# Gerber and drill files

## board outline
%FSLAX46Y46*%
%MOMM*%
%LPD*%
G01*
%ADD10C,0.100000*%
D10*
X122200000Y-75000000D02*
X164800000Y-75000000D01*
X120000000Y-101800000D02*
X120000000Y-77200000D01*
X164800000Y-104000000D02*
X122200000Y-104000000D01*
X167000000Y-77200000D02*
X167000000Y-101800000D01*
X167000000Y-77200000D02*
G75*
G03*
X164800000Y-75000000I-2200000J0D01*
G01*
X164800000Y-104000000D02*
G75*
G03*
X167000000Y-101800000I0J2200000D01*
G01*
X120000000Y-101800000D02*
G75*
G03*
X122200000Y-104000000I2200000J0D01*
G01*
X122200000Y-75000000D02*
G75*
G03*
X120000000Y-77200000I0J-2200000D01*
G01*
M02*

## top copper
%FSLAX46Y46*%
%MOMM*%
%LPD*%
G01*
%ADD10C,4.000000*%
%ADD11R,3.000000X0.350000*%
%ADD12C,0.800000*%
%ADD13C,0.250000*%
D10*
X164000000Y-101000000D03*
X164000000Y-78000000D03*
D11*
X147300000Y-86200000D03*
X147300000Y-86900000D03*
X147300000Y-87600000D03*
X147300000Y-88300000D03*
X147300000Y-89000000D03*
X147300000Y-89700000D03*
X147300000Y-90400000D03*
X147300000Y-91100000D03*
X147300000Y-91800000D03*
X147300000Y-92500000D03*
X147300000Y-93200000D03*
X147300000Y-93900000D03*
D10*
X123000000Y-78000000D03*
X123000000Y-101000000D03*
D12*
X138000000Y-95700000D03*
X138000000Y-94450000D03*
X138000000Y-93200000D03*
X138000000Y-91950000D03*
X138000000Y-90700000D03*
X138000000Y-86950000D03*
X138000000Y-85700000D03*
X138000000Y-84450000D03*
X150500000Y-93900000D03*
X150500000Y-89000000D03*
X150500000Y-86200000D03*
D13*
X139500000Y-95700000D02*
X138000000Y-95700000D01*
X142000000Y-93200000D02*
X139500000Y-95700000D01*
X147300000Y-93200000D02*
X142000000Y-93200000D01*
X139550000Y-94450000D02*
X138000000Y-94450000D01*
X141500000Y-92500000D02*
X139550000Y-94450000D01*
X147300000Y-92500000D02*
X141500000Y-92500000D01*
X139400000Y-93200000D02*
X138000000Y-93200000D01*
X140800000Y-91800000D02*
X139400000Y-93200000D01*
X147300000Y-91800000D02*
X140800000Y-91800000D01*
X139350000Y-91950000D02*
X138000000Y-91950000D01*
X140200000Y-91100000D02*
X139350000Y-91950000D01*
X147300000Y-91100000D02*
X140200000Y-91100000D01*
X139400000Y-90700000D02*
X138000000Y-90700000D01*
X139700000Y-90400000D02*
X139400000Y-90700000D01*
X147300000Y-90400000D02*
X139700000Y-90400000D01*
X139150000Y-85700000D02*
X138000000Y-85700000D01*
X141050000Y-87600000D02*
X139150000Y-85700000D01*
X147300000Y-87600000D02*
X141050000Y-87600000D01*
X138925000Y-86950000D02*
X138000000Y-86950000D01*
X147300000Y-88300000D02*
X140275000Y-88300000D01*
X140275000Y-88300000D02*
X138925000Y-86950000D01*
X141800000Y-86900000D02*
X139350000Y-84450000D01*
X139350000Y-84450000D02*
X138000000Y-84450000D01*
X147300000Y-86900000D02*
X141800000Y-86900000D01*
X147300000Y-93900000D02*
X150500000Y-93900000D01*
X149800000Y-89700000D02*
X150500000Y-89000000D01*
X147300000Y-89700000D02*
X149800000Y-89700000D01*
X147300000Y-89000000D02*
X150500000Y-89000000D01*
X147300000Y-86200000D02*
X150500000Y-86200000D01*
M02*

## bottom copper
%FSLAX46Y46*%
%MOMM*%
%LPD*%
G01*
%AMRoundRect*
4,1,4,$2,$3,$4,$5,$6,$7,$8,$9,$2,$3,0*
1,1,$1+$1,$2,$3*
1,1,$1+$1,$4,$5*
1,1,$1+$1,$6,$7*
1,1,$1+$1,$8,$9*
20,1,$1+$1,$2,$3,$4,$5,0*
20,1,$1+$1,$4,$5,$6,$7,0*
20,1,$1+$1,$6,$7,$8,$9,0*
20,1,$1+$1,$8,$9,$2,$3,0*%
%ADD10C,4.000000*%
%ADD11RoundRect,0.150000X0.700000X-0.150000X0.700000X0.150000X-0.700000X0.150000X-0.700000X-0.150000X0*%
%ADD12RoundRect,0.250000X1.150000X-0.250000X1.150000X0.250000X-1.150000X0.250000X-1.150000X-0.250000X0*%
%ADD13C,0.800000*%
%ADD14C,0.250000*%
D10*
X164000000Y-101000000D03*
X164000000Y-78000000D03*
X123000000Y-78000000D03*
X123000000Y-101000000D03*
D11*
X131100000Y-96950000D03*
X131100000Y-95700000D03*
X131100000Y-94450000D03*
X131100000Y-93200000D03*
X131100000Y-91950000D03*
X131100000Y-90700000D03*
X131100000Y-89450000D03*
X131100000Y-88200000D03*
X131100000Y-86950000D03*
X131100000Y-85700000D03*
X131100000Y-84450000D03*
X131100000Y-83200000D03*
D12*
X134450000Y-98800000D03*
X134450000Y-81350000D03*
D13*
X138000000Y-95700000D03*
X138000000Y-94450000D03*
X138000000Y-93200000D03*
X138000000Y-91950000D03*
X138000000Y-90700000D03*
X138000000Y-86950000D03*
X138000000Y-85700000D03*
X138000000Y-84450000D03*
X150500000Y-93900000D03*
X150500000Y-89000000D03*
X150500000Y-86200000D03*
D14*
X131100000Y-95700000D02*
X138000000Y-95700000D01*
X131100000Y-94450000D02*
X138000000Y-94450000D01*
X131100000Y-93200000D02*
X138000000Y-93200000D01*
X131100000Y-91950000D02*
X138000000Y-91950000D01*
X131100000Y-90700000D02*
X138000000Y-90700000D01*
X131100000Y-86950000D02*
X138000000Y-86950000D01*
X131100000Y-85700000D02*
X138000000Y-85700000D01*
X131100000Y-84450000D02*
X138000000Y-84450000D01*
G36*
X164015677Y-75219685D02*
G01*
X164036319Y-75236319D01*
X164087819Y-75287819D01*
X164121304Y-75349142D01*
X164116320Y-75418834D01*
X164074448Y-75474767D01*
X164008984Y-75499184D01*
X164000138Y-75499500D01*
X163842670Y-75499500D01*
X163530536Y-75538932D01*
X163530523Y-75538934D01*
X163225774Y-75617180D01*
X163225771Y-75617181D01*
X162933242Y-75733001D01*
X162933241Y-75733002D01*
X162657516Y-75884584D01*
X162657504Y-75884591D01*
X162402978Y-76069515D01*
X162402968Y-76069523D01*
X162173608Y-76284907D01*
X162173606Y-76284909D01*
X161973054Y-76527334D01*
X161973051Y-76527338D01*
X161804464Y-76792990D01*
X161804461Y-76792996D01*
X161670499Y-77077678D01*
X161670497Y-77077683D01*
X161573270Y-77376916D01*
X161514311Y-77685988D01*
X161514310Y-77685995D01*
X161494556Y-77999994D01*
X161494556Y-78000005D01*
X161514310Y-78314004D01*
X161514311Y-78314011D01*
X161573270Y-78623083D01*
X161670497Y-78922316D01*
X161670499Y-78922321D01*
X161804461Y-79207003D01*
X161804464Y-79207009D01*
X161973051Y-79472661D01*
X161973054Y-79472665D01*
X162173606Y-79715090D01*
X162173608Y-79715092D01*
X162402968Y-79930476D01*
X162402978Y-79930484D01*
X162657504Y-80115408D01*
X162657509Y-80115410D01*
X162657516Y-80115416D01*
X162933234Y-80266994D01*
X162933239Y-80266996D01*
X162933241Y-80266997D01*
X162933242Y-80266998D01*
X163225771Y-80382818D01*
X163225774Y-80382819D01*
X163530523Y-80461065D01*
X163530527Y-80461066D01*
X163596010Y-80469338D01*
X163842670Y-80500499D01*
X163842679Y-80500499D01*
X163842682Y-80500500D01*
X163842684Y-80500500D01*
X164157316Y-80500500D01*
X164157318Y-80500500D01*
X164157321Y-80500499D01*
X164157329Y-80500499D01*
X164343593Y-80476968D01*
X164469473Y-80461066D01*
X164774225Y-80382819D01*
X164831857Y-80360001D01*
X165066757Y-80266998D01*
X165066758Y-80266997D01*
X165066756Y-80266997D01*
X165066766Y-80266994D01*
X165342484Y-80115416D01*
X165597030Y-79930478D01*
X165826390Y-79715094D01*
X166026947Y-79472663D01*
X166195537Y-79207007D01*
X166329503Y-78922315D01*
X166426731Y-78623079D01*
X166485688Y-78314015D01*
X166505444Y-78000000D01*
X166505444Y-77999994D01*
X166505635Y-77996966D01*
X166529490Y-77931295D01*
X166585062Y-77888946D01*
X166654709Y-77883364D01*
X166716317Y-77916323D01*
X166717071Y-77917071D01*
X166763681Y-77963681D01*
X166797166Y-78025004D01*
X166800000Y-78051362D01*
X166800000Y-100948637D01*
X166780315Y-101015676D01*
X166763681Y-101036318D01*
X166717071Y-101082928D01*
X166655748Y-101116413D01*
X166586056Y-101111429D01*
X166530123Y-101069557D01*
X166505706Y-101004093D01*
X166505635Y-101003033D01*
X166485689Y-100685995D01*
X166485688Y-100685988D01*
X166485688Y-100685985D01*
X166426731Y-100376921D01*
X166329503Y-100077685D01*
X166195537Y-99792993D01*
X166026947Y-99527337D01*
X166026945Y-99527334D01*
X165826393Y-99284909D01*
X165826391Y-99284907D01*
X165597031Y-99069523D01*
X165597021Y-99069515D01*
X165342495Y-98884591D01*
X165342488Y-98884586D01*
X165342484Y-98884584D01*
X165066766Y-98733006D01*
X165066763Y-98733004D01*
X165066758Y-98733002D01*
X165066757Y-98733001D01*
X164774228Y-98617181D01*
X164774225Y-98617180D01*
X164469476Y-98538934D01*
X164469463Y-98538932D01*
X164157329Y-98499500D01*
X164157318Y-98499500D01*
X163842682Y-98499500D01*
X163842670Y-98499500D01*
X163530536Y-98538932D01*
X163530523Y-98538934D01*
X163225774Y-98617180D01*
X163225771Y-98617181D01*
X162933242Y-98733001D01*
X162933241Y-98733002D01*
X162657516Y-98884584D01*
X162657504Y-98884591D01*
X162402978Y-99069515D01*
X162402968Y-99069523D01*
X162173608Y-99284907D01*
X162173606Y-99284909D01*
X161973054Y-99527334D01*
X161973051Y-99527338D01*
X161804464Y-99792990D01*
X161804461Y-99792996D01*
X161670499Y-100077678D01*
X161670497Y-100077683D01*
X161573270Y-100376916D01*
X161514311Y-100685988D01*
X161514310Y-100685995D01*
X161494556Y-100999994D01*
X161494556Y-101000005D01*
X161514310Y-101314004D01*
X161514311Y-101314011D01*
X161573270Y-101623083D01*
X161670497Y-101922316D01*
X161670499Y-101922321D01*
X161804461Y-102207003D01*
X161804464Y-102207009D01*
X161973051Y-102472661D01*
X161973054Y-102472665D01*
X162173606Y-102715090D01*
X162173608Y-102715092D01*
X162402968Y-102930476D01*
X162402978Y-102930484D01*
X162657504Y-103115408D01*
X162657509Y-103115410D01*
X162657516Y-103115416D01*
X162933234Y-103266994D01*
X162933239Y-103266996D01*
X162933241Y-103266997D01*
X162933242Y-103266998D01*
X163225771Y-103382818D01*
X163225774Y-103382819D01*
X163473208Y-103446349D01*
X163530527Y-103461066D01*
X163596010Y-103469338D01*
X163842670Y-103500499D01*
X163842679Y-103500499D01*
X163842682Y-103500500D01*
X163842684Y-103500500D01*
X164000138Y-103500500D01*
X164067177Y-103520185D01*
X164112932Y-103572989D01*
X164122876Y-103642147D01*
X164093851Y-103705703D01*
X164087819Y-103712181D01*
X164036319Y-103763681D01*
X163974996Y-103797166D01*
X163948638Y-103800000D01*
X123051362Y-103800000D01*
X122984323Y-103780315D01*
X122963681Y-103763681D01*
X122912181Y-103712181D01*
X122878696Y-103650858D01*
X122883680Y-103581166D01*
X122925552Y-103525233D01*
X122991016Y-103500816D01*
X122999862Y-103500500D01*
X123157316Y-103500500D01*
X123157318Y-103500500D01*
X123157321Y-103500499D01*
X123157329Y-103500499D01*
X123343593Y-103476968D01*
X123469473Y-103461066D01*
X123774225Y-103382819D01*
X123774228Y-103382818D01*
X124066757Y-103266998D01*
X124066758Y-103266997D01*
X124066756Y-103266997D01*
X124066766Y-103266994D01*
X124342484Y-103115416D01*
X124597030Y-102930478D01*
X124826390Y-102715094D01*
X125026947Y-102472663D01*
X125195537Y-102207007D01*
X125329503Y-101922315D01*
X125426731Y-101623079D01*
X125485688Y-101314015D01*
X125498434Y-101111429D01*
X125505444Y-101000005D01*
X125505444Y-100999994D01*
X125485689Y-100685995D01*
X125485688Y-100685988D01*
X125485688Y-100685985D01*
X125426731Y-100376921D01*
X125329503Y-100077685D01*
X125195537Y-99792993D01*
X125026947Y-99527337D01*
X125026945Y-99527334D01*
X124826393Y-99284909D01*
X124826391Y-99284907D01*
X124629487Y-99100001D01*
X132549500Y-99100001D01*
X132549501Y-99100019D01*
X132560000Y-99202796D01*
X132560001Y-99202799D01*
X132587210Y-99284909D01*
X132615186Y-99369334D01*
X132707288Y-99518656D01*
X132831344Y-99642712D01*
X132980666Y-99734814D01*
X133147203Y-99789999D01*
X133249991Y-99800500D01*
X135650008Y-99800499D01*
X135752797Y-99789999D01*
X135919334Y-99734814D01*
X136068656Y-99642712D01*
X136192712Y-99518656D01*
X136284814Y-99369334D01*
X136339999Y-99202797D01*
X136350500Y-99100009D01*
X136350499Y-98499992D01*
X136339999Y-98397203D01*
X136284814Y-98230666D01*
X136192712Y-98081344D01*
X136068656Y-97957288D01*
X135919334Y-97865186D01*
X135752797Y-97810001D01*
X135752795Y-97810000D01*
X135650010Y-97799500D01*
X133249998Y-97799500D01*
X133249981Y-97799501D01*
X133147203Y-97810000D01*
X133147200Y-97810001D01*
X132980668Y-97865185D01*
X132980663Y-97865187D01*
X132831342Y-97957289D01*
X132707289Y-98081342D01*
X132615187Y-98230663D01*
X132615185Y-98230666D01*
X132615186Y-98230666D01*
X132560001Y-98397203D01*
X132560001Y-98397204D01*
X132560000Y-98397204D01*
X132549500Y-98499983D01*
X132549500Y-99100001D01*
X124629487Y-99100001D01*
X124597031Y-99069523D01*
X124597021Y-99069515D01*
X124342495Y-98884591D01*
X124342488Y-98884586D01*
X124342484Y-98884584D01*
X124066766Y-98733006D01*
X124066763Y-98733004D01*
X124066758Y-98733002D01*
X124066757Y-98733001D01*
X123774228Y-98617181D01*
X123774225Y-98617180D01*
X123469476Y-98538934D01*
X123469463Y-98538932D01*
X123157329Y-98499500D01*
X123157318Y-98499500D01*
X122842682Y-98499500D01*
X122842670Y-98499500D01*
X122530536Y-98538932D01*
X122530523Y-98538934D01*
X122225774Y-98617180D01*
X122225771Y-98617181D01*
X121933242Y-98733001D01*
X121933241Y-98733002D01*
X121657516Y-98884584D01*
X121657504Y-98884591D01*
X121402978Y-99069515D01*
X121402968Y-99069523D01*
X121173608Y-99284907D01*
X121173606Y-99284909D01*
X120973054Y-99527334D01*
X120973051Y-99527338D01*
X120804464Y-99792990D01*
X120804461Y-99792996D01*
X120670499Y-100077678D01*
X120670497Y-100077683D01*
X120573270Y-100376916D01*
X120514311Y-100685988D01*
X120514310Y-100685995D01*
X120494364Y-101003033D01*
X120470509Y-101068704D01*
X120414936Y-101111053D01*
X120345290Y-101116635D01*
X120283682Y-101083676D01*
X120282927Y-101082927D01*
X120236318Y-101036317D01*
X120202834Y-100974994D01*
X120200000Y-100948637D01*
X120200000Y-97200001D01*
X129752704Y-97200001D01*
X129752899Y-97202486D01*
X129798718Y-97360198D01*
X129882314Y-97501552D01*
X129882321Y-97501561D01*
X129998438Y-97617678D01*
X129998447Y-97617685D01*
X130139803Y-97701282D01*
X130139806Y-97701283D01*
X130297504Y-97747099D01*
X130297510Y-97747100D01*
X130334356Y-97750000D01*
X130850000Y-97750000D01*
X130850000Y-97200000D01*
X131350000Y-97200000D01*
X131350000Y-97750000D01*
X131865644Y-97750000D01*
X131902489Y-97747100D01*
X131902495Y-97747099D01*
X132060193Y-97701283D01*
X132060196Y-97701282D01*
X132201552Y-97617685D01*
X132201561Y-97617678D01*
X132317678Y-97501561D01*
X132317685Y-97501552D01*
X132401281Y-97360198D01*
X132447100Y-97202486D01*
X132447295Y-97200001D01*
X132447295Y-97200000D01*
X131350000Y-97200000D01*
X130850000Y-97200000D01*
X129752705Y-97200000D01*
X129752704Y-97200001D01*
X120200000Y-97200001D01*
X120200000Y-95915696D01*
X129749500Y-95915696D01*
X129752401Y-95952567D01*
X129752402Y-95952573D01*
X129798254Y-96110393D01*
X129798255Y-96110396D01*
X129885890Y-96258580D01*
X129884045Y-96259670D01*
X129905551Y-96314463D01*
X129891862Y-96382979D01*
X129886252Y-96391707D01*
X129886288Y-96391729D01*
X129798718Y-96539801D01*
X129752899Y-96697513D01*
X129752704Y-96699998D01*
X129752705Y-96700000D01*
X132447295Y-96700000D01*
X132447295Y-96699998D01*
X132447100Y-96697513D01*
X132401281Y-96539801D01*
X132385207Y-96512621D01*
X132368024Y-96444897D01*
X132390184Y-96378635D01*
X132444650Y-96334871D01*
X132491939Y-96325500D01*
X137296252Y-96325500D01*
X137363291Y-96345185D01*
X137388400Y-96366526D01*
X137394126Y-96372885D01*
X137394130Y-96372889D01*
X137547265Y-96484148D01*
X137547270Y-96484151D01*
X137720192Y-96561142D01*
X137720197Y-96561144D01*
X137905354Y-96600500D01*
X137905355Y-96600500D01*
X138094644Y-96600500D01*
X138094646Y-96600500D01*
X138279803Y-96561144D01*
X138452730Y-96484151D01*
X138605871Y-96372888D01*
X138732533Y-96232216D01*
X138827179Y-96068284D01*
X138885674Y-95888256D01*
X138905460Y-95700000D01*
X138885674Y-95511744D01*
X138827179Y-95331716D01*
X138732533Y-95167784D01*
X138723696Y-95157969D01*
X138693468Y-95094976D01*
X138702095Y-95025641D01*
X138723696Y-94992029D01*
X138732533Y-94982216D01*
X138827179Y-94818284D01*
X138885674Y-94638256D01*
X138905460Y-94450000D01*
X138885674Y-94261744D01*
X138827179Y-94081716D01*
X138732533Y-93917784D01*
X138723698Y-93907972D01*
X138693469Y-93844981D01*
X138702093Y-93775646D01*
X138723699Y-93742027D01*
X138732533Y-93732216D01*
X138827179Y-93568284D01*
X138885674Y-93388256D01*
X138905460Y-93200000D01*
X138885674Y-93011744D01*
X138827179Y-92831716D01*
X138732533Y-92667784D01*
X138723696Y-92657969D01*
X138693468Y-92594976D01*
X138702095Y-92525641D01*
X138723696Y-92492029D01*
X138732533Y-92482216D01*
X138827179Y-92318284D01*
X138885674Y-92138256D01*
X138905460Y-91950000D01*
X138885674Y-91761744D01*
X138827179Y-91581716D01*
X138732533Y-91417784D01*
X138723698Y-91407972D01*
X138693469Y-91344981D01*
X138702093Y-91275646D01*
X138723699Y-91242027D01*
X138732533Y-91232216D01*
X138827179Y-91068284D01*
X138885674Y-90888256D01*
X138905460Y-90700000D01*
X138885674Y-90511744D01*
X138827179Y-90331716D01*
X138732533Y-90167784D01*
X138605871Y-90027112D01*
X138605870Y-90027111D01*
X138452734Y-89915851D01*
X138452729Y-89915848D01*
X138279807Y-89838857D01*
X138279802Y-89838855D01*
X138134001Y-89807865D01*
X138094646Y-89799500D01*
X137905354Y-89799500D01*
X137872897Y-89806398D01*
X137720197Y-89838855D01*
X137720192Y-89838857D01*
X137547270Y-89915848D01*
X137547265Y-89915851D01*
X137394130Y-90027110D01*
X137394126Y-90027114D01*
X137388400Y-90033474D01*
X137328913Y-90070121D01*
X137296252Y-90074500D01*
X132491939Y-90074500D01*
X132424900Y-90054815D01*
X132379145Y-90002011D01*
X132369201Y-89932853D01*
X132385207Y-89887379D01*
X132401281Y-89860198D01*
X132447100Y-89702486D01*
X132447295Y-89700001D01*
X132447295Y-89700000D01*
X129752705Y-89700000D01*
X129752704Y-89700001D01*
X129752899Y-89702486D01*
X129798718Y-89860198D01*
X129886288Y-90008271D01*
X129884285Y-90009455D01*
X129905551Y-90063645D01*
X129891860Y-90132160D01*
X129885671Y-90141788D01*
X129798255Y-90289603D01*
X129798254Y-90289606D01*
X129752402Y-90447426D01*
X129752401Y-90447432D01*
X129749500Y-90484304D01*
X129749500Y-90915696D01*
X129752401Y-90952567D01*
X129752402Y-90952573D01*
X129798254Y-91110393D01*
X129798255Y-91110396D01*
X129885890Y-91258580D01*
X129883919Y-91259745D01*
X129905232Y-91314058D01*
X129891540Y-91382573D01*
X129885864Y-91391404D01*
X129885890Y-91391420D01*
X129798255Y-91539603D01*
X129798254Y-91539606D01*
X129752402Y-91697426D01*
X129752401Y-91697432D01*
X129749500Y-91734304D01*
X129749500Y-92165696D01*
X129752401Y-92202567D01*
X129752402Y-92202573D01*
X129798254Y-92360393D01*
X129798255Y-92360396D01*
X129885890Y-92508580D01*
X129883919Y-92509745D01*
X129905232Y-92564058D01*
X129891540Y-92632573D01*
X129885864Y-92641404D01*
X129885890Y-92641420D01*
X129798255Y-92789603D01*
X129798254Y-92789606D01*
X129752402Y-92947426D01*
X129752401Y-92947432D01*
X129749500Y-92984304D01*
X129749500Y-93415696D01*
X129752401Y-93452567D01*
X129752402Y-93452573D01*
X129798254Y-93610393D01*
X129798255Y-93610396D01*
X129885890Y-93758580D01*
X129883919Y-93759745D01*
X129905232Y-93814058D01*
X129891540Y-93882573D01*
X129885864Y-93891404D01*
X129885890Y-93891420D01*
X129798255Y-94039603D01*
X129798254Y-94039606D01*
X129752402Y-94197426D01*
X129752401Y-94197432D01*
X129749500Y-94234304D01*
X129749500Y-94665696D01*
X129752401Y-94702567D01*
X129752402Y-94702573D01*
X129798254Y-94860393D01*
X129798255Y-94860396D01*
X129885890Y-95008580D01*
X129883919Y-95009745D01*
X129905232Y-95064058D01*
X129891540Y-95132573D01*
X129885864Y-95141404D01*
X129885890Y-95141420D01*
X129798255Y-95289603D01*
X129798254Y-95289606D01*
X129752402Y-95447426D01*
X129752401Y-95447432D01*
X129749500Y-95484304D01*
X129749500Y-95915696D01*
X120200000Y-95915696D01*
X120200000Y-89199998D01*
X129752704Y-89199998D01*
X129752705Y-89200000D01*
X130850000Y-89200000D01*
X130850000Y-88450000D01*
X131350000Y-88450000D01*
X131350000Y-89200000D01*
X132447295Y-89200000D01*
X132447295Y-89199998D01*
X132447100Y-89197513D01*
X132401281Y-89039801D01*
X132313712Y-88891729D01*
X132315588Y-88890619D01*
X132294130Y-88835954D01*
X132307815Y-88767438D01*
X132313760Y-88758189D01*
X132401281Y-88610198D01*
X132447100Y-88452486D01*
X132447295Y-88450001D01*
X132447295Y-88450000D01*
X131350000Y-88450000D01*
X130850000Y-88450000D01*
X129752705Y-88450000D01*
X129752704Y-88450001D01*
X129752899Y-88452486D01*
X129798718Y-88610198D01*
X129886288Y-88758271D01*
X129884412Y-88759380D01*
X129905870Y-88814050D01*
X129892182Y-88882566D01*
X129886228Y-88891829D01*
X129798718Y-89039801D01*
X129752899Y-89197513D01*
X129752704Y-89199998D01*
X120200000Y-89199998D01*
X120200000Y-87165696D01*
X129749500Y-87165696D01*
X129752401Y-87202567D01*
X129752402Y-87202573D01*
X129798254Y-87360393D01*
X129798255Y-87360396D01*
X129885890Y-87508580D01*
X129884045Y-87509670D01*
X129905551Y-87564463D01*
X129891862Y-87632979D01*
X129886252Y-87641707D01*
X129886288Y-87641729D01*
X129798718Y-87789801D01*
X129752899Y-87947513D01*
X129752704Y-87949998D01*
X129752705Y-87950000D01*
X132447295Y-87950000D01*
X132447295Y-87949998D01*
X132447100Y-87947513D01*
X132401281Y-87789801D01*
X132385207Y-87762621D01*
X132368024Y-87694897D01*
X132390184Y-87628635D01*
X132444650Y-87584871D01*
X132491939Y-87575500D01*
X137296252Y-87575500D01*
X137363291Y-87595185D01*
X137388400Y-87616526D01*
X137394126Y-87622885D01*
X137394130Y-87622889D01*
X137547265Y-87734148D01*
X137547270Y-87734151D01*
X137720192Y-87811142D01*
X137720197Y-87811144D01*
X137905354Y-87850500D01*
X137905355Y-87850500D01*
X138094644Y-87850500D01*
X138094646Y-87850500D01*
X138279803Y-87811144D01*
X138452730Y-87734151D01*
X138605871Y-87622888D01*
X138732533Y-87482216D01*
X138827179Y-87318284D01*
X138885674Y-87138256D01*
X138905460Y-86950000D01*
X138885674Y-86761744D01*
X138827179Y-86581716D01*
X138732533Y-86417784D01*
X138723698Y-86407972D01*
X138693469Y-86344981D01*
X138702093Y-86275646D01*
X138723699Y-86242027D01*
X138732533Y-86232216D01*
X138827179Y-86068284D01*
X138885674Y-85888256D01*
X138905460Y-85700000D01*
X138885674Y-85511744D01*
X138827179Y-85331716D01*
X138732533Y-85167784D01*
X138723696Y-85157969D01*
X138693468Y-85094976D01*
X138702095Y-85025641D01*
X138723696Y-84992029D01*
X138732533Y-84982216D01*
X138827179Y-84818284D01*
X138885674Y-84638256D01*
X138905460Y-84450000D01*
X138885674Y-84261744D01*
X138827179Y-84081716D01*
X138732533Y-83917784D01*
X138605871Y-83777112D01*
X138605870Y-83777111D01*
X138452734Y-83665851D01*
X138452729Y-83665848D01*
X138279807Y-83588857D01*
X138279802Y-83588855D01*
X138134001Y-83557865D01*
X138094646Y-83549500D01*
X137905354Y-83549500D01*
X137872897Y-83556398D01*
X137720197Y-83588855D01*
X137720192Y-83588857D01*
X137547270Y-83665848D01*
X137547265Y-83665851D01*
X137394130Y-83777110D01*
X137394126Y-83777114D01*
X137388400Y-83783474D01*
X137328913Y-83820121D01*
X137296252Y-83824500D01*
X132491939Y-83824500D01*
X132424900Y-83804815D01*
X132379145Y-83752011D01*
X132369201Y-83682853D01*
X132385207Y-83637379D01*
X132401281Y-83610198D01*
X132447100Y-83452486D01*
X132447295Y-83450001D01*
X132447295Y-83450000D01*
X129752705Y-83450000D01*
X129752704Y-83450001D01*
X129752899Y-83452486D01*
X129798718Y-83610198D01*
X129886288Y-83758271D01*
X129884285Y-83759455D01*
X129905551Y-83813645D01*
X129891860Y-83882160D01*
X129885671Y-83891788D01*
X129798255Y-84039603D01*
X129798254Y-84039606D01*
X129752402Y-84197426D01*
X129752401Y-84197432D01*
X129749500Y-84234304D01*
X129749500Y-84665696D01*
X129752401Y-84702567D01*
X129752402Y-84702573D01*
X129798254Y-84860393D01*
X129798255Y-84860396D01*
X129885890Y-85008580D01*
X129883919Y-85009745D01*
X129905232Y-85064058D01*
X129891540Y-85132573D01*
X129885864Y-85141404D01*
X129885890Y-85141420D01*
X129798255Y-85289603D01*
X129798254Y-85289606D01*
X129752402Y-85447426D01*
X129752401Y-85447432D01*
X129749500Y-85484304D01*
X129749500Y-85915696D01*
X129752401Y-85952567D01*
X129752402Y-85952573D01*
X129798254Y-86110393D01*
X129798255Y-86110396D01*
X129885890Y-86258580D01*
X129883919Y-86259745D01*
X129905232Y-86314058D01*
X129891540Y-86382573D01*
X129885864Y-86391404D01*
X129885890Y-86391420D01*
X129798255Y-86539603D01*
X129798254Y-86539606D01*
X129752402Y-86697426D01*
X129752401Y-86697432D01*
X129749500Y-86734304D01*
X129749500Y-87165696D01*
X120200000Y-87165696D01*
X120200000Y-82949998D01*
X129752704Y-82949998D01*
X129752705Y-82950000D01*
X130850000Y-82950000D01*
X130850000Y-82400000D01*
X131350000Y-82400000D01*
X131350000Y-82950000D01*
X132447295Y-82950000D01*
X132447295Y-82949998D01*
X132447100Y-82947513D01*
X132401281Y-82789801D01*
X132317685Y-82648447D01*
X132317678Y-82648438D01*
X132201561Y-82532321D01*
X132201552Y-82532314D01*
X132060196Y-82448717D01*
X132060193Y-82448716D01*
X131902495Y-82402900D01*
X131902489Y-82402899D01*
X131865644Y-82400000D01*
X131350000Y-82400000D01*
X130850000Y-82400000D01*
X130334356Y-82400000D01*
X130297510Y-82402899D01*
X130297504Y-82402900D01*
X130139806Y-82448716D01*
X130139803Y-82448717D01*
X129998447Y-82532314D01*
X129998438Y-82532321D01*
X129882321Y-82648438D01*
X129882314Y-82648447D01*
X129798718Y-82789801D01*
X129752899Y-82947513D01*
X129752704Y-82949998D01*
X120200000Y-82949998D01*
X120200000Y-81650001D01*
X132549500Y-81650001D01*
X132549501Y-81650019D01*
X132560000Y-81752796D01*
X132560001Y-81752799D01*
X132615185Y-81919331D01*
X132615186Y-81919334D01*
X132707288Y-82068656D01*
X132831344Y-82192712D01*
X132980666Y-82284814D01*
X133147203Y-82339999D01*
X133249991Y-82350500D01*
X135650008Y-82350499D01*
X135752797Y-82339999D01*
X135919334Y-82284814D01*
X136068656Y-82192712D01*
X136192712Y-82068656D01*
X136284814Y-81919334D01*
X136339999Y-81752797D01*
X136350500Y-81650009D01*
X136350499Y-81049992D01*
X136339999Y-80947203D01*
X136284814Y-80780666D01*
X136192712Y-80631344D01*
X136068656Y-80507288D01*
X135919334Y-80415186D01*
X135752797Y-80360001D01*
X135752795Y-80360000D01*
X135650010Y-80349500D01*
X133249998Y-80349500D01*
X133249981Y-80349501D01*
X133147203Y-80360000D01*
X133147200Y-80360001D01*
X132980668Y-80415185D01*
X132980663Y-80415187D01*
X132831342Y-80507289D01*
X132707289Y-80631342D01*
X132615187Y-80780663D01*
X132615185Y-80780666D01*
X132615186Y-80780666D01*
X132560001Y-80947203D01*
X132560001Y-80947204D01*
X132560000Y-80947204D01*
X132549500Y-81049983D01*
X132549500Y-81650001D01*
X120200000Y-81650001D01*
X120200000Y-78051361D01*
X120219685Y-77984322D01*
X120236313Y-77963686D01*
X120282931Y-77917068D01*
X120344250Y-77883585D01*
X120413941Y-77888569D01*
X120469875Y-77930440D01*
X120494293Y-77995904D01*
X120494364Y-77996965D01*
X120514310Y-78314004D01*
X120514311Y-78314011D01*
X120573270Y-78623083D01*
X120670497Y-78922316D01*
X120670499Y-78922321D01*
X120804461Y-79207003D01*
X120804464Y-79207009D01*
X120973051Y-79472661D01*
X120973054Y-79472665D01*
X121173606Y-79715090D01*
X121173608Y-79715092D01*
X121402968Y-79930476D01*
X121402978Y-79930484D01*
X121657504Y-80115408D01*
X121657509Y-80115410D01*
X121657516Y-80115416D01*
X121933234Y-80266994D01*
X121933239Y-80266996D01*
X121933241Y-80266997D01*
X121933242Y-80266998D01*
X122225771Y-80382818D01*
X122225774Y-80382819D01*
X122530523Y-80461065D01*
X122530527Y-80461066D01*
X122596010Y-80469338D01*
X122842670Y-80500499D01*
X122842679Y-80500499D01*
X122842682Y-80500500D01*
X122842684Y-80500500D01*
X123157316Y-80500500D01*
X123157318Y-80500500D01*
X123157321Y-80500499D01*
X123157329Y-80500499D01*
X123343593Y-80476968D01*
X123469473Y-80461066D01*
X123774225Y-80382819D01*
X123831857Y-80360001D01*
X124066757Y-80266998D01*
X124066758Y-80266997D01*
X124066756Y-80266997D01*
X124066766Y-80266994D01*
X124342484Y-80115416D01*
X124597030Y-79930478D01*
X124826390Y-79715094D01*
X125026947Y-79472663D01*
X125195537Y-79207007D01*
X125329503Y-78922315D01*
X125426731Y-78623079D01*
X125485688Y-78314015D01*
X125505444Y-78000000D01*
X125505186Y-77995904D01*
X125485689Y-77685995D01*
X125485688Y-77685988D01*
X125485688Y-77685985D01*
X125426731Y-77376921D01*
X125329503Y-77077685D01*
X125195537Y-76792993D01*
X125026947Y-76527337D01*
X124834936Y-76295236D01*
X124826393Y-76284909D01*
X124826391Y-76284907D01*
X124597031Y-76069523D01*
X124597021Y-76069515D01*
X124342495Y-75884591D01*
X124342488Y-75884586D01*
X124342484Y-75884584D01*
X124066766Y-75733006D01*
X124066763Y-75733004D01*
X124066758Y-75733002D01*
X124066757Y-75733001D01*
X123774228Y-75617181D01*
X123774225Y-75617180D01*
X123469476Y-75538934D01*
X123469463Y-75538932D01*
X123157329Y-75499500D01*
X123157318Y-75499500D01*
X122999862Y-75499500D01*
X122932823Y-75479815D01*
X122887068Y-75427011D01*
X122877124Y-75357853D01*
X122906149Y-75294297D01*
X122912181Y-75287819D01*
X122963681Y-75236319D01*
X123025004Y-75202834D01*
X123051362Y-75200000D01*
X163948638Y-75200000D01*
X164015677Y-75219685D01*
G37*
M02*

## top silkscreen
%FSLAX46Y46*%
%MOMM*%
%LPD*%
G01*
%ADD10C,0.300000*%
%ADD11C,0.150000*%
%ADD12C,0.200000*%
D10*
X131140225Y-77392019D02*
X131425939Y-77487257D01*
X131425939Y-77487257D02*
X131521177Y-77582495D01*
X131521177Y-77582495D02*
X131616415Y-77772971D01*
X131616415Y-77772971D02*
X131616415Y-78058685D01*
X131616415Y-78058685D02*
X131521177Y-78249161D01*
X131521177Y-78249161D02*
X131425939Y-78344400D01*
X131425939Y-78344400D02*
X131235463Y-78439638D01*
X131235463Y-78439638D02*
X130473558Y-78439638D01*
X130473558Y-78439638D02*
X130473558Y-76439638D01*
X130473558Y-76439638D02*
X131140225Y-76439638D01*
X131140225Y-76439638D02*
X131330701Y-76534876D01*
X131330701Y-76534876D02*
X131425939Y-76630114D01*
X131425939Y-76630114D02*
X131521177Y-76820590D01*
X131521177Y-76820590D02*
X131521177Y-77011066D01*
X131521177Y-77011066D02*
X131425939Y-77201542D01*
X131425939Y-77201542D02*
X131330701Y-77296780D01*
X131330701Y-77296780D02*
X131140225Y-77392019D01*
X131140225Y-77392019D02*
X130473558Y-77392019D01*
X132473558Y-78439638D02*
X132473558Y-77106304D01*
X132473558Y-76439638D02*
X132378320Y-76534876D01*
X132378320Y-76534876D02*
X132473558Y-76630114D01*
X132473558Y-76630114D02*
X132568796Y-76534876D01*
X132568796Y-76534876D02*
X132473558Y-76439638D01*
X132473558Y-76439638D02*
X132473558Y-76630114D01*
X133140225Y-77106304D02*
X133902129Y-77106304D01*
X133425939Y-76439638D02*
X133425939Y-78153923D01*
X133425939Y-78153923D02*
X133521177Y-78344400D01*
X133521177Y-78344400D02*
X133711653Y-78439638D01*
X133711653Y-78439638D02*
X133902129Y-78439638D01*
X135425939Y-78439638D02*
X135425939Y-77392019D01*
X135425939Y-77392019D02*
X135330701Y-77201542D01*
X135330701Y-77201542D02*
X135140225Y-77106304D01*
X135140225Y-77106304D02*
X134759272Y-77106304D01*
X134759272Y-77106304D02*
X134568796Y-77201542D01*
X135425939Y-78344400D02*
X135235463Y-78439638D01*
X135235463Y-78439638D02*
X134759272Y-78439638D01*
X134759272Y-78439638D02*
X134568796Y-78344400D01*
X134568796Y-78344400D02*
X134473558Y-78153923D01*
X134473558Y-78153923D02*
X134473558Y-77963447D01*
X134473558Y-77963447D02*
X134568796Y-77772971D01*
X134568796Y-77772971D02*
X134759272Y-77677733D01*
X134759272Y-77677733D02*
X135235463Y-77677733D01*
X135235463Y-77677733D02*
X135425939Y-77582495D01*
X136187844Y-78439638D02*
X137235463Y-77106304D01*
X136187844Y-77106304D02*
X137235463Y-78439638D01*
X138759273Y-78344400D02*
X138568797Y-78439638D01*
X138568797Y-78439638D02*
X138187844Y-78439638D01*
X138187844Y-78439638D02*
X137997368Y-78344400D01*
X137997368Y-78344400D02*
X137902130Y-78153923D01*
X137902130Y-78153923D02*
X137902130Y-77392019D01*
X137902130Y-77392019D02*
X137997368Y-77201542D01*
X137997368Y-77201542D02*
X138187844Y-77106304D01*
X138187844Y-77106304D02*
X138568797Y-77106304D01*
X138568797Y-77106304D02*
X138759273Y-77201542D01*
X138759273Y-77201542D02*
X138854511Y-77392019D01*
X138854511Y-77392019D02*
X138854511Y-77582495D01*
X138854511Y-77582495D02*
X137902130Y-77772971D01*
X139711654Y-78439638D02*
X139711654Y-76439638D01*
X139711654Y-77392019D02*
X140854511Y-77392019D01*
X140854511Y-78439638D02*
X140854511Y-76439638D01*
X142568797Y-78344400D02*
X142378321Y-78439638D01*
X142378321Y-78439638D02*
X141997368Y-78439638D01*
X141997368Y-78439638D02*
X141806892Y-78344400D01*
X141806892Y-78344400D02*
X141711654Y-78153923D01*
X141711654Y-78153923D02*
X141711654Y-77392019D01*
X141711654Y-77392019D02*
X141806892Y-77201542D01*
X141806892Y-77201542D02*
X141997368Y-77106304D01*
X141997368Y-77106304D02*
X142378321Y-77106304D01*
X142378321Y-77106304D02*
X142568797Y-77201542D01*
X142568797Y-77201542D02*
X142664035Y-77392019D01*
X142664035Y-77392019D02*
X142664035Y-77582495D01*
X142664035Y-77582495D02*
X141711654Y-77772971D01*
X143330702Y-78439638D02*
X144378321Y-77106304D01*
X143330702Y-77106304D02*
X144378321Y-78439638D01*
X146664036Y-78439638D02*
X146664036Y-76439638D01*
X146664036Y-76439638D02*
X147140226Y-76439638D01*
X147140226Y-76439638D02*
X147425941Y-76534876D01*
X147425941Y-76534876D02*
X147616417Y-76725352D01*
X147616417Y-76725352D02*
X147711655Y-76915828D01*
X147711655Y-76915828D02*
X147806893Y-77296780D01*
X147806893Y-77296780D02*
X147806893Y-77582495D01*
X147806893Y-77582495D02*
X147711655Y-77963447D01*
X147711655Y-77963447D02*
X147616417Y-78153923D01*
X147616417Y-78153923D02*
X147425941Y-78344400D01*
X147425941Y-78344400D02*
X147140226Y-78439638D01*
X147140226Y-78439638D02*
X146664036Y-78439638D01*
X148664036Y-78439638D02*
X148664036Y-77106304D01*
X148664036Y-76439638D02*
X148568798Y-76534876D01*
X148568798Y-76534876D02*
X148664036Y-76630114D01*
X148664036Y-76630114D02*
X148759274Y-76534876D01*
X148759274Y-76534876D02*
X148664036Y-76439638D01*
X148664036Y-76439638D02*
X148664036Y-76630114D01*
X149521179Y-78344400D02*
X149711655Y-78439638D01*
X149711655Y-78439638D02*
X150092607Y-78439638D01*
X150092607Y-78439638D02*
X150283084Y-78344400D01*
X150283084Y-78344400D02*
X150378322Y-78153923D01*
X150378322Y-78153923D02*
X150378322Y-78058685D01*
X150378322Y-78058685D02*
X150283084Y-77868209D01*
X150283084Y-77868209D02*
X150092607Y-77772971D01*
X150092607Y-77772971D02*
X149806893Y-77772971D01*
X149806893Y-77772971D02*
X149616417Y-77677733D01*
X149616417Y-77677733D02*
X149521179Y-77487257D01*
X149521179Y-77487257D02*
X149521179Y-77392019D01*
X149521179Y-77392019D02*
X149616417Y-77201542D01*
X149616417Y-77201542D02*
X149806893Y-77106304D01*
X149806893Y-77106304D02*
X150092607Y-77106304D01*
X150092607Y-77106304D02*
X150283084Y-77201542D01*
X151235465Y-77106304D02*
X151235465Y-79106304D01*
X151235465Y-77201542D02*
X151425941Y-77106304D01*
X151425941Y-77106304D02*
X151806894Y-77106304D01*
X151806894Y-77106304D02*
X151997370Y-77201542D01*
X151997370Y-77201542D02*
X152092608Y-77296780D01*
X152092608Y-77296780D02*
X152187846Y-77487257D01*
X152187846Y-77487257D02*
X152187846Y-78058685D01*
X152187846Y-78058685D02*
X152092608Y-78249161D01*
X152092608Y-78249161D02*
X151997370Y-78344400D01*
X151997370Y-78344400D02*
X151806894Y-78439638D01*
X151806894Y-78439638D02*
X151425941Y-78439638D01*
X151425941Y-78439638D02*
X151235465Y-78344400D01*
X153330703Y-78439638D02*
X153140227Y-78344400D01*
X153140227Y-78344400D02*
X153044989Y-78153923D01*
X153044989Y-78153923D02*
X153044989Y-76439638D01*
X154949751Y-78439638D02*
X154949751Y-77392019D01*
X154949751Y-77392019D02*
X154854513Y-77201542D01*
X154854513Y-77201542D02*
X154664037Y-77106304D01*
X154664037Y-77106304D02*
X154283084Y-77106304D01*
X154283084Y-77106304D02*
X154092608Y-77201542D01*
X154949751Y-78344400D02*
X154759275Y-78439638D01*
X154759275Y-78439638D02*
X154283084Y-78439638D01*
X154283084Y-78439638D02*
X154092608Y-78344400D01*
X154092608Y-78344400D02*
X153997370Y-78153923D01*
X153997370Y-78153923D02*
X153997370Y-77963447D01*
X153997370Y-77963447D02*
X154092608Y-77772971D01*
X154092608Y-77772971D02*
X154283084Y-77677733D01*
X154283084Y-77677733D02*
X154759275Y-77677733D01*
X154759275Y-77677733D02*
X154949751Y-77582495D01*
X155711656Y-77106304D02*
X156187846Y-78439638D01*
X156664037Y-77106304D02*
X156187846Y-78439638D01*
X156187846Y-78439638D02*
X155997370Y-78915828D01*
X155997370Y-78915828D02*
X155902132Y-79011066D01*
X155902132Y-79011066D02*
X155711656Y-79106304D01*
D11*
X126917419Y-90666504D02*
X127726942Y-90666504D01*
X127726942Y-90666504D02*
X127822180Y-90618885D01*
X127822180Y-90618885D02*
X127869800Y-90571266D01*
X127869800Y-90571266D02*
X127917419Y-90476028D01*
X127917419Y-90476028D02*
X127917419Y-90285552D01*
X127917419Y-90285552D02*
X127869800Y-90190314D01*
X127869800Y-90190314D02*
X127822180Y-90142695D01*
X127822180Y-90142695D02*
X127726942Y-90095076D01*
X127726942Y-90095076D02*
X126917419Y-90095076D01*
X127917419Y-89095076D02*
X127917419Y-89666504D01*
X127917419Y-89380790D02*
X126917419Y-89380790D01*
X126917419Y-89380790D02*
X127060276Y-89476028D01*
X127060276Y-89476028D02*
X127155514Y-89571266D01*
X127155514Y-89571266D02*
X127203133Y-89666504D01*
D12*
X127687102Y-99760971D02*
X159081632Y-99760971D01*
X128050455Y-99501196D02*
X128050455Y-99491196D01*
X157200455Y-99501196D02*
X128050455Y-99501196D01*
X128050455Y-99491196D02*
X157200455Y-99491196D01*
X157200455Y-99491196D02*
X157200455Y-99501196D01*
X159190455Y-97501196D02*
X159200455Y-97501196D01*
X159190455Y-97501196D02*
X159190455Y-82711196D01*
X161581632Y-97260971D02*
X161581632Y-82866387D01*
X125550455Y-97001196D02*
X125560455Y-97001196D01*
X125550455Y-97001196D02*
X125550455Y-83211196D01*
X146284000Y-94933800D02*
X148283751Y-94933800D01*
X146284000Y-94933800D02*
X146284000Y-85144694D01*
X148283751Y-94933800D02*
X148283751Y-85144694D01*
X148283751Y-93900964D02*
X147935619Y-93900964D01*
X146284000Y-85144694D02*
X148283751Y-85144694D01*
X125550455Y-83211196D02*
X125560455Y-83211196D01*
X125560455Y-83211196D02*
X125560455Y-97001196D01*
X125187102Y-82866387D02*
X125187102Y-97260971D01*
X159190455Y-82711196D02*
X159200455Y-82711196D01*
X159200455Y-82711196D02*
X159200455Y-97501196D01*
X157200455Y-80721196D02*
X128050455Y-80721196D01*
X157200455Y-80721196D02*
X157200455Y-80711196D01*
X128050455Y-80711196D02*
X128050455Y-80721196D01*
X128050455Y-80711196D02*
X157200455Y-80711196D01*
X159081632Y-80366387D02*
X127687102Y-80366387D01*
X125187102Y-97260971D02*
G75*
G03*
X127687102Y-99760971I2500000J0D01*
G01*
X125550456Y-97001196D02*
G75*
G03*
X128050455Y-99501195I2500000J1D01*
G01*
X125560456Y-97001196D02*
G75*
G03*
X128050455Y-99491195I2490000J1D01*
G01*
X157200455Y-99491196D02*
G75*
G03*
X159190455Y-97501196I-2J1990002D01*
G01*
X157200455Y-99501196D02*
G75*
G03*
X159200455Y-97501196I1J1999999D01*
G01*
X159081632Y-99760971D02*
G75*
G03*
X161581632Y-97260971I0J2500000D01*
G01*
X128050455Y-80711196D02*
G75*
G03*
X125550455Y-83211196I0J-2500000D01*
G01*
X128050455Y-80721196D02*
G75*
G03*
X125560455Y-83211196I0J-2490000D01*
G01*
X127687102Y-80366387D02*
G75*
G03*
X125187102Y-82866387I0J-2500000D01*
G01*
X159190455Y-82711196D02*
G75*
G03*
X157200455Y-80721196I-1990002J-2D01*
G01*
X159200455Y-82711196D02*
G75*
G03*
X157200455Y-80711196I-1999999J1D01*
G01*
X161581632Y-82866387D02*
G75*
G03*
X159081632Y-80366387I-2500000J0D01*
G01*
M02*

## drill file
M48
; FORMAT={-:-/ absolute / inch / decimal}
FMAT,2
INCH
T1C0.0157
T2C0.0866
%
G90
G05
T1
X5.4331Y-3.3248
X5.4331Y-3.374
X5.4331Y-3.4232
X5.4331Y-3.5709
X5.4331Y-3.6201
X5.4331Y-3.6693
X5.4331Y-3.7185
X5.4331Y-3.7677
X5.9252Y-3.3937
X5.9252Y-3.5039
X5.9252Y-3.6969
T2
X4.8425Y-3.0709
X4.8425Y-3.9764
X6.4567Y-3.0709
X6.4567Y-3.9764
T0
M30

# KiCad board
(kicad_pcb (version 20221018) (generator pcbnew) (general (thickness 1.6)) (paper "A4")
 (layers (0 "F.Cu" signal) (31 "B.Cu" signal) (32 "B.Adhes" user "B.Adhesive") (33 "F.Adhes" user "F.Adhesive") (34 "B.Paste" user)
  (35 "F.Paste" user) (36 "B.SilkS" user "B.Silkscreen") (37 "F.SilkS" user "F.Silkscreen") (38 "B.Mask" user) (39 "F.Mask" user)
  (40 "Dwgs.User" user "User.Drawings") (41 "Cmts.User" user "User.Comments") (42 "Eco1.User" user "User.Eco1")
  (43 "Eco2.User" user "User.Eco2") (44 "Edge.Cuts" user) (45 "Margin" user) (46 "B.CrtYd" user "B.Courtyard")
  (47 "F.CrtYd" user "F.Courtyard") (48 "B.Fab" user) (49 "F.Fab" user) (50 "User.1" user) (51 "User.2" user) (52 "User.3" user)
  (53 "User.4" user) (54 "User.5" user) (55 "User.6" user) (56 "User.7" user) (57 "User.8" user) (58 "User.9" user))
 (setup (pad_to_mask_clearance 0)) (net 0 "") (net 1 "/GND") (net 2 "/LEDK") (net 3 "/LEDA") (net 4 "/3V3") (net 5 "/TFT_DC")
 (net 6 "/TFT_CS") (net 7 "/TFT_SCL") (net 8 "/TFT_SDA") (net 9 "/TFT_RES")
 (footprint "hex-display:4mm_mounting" (layer "F.Cu") (at 164.1 101.2)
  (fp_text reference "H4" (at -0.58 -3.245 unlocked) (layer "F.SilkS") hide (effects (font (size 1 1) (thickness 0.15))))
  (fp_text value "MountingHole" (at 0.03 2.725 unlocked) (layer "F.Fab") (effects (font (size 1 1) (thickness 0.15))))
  (pad "" thru_hole circle (at -0.1 -0.2) (size 4 4) (drill 2.2) (layers "*.Cu" "*.Mask") (zone_connect 0)))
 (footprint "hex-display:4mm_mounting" (layer "F.Cu") (at 163.6 78.2)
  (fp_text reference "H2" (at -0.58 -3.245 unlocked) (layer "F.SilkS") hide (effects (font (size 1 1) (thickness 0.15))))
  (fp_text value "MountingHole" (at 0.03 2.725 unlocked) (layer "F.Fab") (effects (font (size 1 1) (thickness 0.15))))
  (pad "" thru_hole circle (at 0.4 -0.2) (size 4 4) (drill 2.2) (layers "*.Cu" "*.Mask") (zone_connect 0)))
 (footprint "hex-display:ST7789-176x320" (layer "F.Cu") (at 172.954 65.7238 90)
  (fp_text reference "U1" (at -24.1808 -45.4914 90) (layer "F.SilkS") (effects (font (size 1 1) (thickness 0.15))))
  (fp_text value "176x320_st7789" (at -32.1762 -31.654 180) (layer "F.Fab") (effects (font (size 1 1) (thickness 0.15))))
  (fp_line (start -34.037171 -45.266898) (end -34.037171 -13.872368) (stroke (width 0.2) (type solid)) (layer "F.SilkS"))
  (fp_line (start -33.777396 -44.903545) (end -33.767396 -44.903545) (stroke (width 0.2) (type solid)) (layer "F.SilkS"))
  (fp_line (start -33.777396 -15.753545) (end -33.777396 -44.903545) (stroke (width 0.2) (type solid)) (layer "F.SilkS"))
  (fp_line (start -33.767396 -44.903545) (end -33.767396 -15.753545) (stroke (width 0.2) (type solid)) (layer "F.SilkS"))
  (fp_line (start -33.767396 -15.753545) (end -33.777396 -15.753545) (stroke (width 0.2) (type solid)) (layer "F.SilkS"))
  (fp_line (start -31.777396 -13.763545) (end -31.777396 -13.753545) (stroke (width 0.2) (type solid)) (layer "F.SilkS"))
  (fp_line (start -31.777396 -13.763545) (end -16.987396 -13.763545) (stroke (width 0.2) (type solid)) (layer "F.SilkS"))
  (fp_line (start -31.537171 -11.372368) (end -17.142587 -11.372368) (stroke (width 0.2) (type solid)) (layer "F.SilkS"))
  (fp_line (start -31.277396 -47.403545) (end -31.277396 -47.393545) (stroke (width 0.2) (type solid)) (layer "F.SilkS"))
  (fp_line (start -31.277396 -47.403545) (end -17.487396 -47.403545) (stroke (width 0.2) (type solid)) (layer "F.SilkS"))
  (fp_line (start -29.21 -26.67) (end -29.21 -24.670249) (stroke (width 0.2) (type solid)) (layer "F.SilkS"))
  (fp_line (start -29.21 -26.67) (end -19.420894 -26.67) (stroke (width 0.2) (type solid)) (layer "F.SilkS"))
  (fp_line (start -29.21 -24.670249) (end -19.420894 -24.670249) (stroke (width 0.2) (type solid)) (layer "F.SilkS"))
  (fp_line (start -28.177164 -24.670249) (end -28.177164 -25.018381) (stroke (width 0.2) (type solid)) (layer "F.SilkS"))
  (fp_line (start -19.420894 -26.67) (end -19.420894 -24.670249) (stroke (width 0.2) (type solid)) (layer "F.SilkS"))
  (fp_line (start -17.487396 -47.403545) (end -17.487396 -47.393545) (stroke (width 0.2) (type solid)) (layer "F.SilkS"))
  (fp_line (start -17.487396 -47.393545) (end -31.277396 -47.393545) (stroke (width 0.2) (type solid)) (layer "F.SilkS"))
  (fp_line (start -17.142587 -47.766898) (end -31.537171 -47.766898) (stroke (width 0.2) (type solid)) (layer "F.SilkS"))
  (fp_line (start -16.987396 -13.763545) (end -16.987396 -13.753545) (stroke (width 0.2) (type solid)) (layer "F.SilkS"))
  (fp_line (start -16.987396 -13.753545) (end -31.777396 -13.753545) (stroke (width 0.2) (type solid)) (layer "F.SilkS"))
  (fp_line (start -14.997396 -15.753545) (end -14.997396 -44.903545) (stroke (width 0.2) (type solid)) (layer "F.SilkS"))
  (fp_line (start -14.997396 -15.753545) (end -14.987396 -15.753545) (stroke (width 0.2) (type solid)) (layer "F.SilkS"))
  (fp_line (start -14.987396 -44.903545) (end -14.997396 -44.903545) (stroke (width 0.2) (type solid)) (layer "F.SilkS"))
  (fp_line (start -14.987396 -44.903545) (end -14.987396 -15.753545) (stroke (width 0.2) (type solid)) (layer "F.SilkS"))
  (fp_line (start -14.642587 -13.872368) (end -14.642587 -45.266898) (stroke (width 0.2) (type solid)) (layer "F.SilkS"))
  (fp_arc (start -34.037171 -45.266898) (mid -33.304938 -47.034665) (end -31.537171 -47.766898) (stroke (width 0.2) (type solid))
   (layer "F.SilkS"))
  (fp_arc (start -33.777395 -44.903545) (mid -33.045162 -46.671311) (end -31.277396 -47.403544) (stroke (width 0.2) (type solid))
   (layer "F.SilkS"))
  (fp_arc (start -33.767395 -44.903545) (mid -33.038091 -46.66424) (end -31.277396 -47.393544) (stroke (width 0.2) (type solid))
   (layer "F.SilkS"))
  (fp_arc (start -31.777396 -13.763545) (mid -33.184538 -14.346403) (end -33.767396 -15.753545) (stroke (width 0.2) (type solid))
   (layer "F.SilkS"))
  (fp_arc (start -31.777396 -13.753545) (mid -33.19161 -14.339331) (end -33.777396 -15.753545) (stroke (width 0.2) (type solid))
   (layer "F.SilkS"))
  (fp_arc (start -31.537171 -11.372368) (mid -33.304938 -12.104601) (end -34.037171 -13.872368) (stroke (width 0.2) (type solid))
   (layer "F.SilkS"))
  (fp_arc (start -17.487396 -47.403545) (mid -15.719629 -46.671312) (end -14.987396 -44.903545) (stroke (width 0.2) (type solid))
   (layer "F.SilkS"))
  (fp_arc (start -17.487396 -47.393545) (mid -15.7267 -46.664241) (end -14.997396 -44.903545) (stroke (width 0.2) (type solid))
   (layer "F.SilkS"))
  (fp_arc (start -17.142587 -47.766898) (mid -15.37482 -47.034665) (end -14.642587 -45.266898) (stroke (width 0.2) (type solid))
   (layer "F.SilkS"))
  (fp_arc (start -14.997396 -15.753545) (mid -15.580254 -14.346403) (end -16.987396 -13.763545) (stroke (width 0.2) (type solid))
   (layer "F.SilkS"))
  (fp_arc (start -14.987396 -15.753545) (mid -15.573182 -14.339331) (end -16.987396 -13.753545) (stroke (width 0.2) (type solid))
   (layer "F.SilkS"))
  (fp_arc (start -14.642587 -13.872368) (mid -15.37482 -12.104601) (end -17.142587 -11.372368) (stroke (width 0.2) (type solid))
   (layer "F.SilkS"))
  (pad "1" smd rect (at -20.4762 -25.654 270) (size 0.35 3) (layers "F.Cu" "F.Paste" "F.Mask") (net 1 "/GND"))
  (pad "2" smd rect (at -21.1762 -25.654 270) (size 0.35 3) (layers "F.Cu" "F.Paste" "F.Mask") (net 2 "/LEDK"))
  (pad "3" smd rect (at -21.8762 -25.654 270) (size 0.35 3) (layers "F.Cu" "F.Paste" "F.Mask") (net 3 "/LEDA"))
  (pad "4" smd rect (at -22.5762 -25.654 270) (size 0.35 3) (layers "F.Cu" "F.Paste" "F.Mask") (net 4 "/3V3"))
  (pad "5" smd rect (at -23.2762 -25.654 270) (size 0.35 3) (layers "F.Cu" "F.Paste" "F.Mask") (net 1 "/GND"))
  (pad "6" smd rect (at -23.9762 -25.654 270) (size 0.35 3) (layers "F.Cu" "F.Paste" "F.Mask") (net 1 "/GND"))
  (pad "7" smd rect (at -24.6762 -25.654 270) (size 0.35 3) (layers "F.Cu" "F.Paste" "F.Mask") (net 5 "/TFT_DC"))
  (pad "8" smd rect (at -25.3762 -25.654 270) (size 0.35 3) (layers "F.Cu" "F.Paste" "F.Mask") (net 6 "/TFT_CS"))
  (pad "9" smd rect (at -26.0762 -25.654 270) (size 0.35 3) (layers "F.Cu" "F.Paste" "F.Mask") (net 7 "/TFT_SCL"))
  (pad "10" smd rect (at -26.7762 -25.654 270) (size 0.35 3) (layers "F.Cu" "F.Paste" "F.Mask") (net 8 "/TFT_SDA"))
  (pad "11" smd rect (at -27.4762 -25.654 270) (size 0.35 3) (layers "F.Cu" "F.Paste" "F.Mask") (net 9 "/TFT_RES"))
  (pad "12" smd rect (at -28.1762 -25.654 270) (size 0.35 3) (layers "F.Cu" "F.Paste" "F.Mask") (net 1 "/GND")))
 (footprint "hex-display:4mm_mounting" (layer "F.Cu") (at 123 78)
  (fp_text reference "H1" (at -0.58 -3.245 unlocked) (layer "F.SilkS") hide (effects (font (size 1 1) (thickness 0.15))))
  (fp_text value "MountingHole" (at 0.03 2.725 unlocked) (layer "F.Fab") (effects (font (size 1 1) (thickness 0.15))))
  (pad "" thru_hole circle (at 0 0) (size 4 4) (drill 2.2) (layers "*.Cu" "*.Mask") (zone_connect 0)))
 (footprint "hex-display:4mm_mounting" (layer "F.Cu") (at 122.9 101)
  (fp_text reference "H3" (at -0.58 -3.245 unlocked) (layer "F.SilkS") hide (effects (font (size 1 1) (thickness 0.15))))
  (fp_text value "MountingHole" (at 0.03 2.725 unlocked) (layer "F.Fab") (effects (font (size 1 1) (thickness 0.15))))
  (pad "" thru_hole circle (at 0.1 0) (size 4 4) (drill 2.2) (layers "*.Cu" "*.Mask") (zone_connect 0)))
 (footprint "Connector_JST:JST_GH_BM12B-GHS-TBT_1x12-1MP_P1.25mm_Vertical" (layer "B.Cu") (at 133.05 90.075 90)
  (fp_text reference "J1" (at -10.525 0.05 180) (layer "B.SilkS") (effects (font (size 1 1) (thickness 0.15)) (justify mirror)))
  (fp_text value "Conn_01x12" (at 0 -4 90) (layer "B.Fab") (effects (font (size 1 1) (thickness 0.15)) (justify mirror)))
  (pad "1" smd roundrect (at -6.875 -1.95 90) (size 0.6 1.7) (layers "B.Cu" "B.Paste" "B.Mask") (roundrect_rratio 0.25) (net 1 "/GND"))
  (pad "2" smd roundrect (at -5.625 -1.95 90) (size 0.6 1.7) (layers "B.Cu" "B.Paste" "B.Mask") (roundrect_rratio 0.25) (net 9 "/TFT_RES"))
  (pad "3" smd roundrect (at -4.375 -1.95 90) (size 0.6 1.7) (layers "B.Cu" "B.Paste" "B.Mask") (roundrect_rratio 0.25) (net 8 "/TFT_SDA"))
  (pad "4" smd roundrect (at -3.125 -1.95 90) (size 0.6 1.7) (layers "B.Cu" "B.Paste" "B.Mask") (roundrect_rratio 0.25) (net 7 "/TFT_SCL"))
  (pad "5" smd roundrect (at -1.875 -1.95 90) (size 0.6 1.7) (layers "B.Cu" "B.Paste" "B.Mask") (roundrect_rratio 0.25) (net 6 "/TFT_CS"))
  (pad "6" smd roundrect (at -0.625 -1.95 90) (size 0.6 1.7) (layers "B.Cu" "B.Paste" "B.Mask") (roundrect_rratio 0.25) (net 5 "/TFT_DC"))
  (pad "7" smd roundrect (at 0.625 -1.95 90) (size 0.6 1.7) (layers "B.Cu" "B.Paste" "B.Mask") (roundrect_rratio 0.25) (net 1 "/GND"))
  (pad "8" smd roundrect (at 1.875 -1.95 90) (size 0.6 1.7) (layers "B.Cu" "B.Paste" "B.Mask") (roundrect_rratio 0.25) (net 1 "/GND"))
  (pad "9" smd roundrect (at 3.125 -1.95 90) (size 0.6 1.7) (layers "B.Cu" "B.Paste" "B.Mask") (roundrect_rratio 0.25) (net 4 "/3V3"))
  (pad "10" smd roundrect (at 4.375 -1.95 90) (size 0.6 1.7) (layers "B.Cu" "B.Paste" "B.Mask") (roundrect_rratio 0.25) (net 3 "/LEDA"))
  (pad "11" smd roundrect (at 5.625 -1.95 90) (size 0.6 1.7) (layers "B.Cu" "B.Paste" "B.Mask") (roundrect_rratio 0.25) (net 2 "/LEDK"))
  (pad "12" smd roundrect (at 6.875 -1.95 90) (size 0.6 1.7) (layers "B.Cu" "B.Paste" "B.Mask") (roundrect_rratio 0.25) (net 1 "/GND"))
  (pad "MP" smd roundrect (at -8.725 1.4 90) (size 1 2.8) (layers "B.Cu" "B.Paste" "B.Mask") (roundrect_rratio 0.25))
  (pad "MP" smd roundrect (at 8.725 1.4 90) (size 1 2.8) (layers "B.Cu" "B.Paste" "B.Mask") (roundrect_rratio 0.25)))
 (gr_line (start 122.2 75) (end 164.8 75) (stroke (width 0.1) (type default)) (layer "Edge.Cuts"))
 (gr_arc (start 122.2 104) (mid 120.644365 103.355635) (end 120 101.8) (stroke (width 0.1) (type default)) (layer "Edge.Cuts"))
 (gr_line (start 167 77.2) (end 167 101.8) (stroke (width 0.1) (type default)) (layer "Edge.Cuts"))
 (gr_arc (start 167 101.8) (mid 166.355635 103.355635) (end 164.8 104) (stroke (width 0.1) (type default)) (layer "Edge.Cuts"))
 (gr_arc (start 164.8 75) (mid 166.355635 75.644365) (end 167 77.2) (stroke (width 0.1) (type default)) (layer "Edge.Cuts"))
 (gr_arc (start 120 77.2) (mid 120.644365 75.644365) (end 122.2 75) (stroke (width 0.1) (type default)) (layer "Edge.Cuts"))
 (gr_line (start 164.8 104) (end 122.2 104) (stroke (width 0.1) (type default)) (layer "Edge.Cuts"))
 (gr_line (start 120 101.8) (end 120 77.2) (stroke (width 0.1) (type default)) (layer "Edge.Cuts"))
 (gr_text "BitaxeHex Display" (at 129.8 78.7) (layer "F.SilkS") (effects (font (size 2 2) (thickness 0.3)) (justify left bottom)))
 (segment (start 147.3 89) (end 150.5 89) (width 0.25) (layer "F.Cu") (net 1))
 (segment (start 149.8 89.7) (end 150.5 89) (width 0.25) (layer "F.Cu") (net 1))
 (segment (start 147.3 93.9) (end 150.5 93.9) (width 0.25) (layer "F.Cu") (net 1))
 (segment (start 147.3 89.7) (end 149.8 89.7) (width 0.25) (layer "F.Cu") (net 1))
 (segment (start 147.3 86.2) (end 150.5 86.2) (width 0.25) (layer "F.Cu") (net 1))
 (via (at 150.5 86.2) (size 0.8) (drill 0.4) (layers "F.Cu" "B.Cu") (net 1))
 (via (at 150.5 93.9) (size 0.8) (drill 0.4) (layers "F.Cu" "B.Cu") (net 1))
 (via (at 150.5 89) (size 0.8) (drill 0.4) (layers "F.Cu" "B.Cu") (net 1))
 (segment (start 142 93.2) (end 139.5 95.7) (width 0.25) (layer "F.Cu") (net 9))
 (segment (start 139.5 95.7) (end 138 95.7) (width 0.25) (layer "F.Cu") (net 9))
 (segment (start 147.3 93.2) (end 142 93.2) (width 0.25) (layer "F.Cu") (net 9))
 (via (at 138 95.7) (size 0.8) (drill 0.4) (layers "F.Cu" "B.Cu") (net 9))
 (segment (start 131.1 95.7) (end 138 95.7) (width 0.25) (layer "B.Cu") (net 9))
 (segment (start 141.5 92.5) (end 139.55 94.45) (width 0.25) (layer "F.Cu") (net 8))
 (segment (start 139.55 94.45) (end 138 94.45) (width 0.25) (layer "F.Cu") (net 8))
 (segment (start 147.3 92.5) (end 141.5 92.5) (width 0.25) (layer "F.Cu") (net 8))
 (via (at 138 94.45) (size 0.8) (drill 0.4) (layers "F.Cu" "B.Cu") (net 8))
 (segment (start 131.1 94.45) (end 138 94.45) (width 0.25) (layer "B.Cu") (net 8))
 (segment (start 147.3 91.8) (end 140.8 91.8) (width 0.25) (layer "F.Cu") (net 7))
 (segment (start 139.4 93.2) (end 138 93.2) (width 0.25) (layer "F.Cu") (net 7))
 (segment (start 140.8 91.8) (end 139.4 93.2) (width 0.25) (layer "F.Cu") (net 7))
 (via (at 138 93.2) (size 0.8) (drill 0.4) (layers "F.Cu" "B.Cu") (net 7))
 (segment (start 131.1 93.2) (end 138 93.2) (width 0.25) (layer "B.Cu") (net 7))
 (segment (start 140.2 91.1) (end 139.35 91.95) (width 0.25) (layer "F.Cu") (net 6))
 (segment (start 147.3 91.1) (end 140.2 91.1) (width 0.25) (layer "F.Cu") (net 6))
 (segment (start 139.35 91.95) (end 138 91.95) (width 0.25) (layer "F.Cu") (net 6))
 (via (at 138 91.95) (size 0.8) (drill 0.4) (layers "F.Cu" "B.Cu") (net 6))
 (segment (start 131.1 91.95) (end 138 91.95) (width 0.25) (layer "B.Cu") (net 6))
 (segment (start 139.7 90.4) (end 139.4 90.7) (width 0.25) (layer "F.Cu") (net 5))
 (segment (start 139.4 90.7) (end 138 90.7) (width 0.25) (layer "F.Cu") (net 5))
 (segment (start 147.3 90.4) (end 139.7 90.4) (width 0.25) (layer "F.Cu") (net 5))
 (via (at 138 90.7) (size 0.8) (drill 0.4) (layers "F.Cu" "B.Cu") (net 5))
 (segment (start 131.1 90.7) (end 138 90.7) (width 0.25) (layer "B.Cu") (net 5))
 (segment (start 138.925 86.95) (end 138 86.95) (width 0.25) (layer "F.Cu") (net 4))
 (segment (start 140.275 88.3) (end 138.925 86.95) (width 0.25) (layer "F.Cu") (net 4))
 (segment (start 147.3 88.3) (end 140.275 88.3) (width 0.25) (layer "F.Cu") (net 4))
 (via (at 138 86.95) (size 0.8) (drill 0.4) (layers "F.Cu" "B.Cu") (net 4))
 (segment (start 131.1 86.95) (end 138 86.95) (width 0.25) (layer "B.Cu") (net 4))
 (segment (start 139.15 85.7) (end 138 85.7) (width 0.25) (layer "F.Cu") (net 3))
 (segment (start 147.3 87.6) (end 141.05 87.6) (width 0.25) (layer "F.Cu") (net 3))
 (segment (start 141.05 87.6) (end 139.15 85.7) (width 0.25) (layer "F.Cu") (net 3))
 (via (at 138 85.7) (size 0.8) (drill 0.4) (layers "F.Cu" "B.Cu") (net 3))
 (segment (start 131.1 85.7) (end 138 85.7) (width 0.25) (layer "B.Cu") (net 3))
 (segment (start 147.3 86.9) (end 141.8 86.9) (width 0.25) (layer "F.Cu") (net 2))
 (segment (start 139.35 84.45) (end 138 84.45) (width 0.25) (layer "F.Cu") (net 2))
 (segment (start 141.8 86.9) (end 139.35 84.45) (width 0.25) (layer "F.Cu") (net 2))
 (via (at 138 84.45) (size 0.8) (drill 0.4) (layers "F.Cu" "B.Cu") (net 2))
 (segment (start 131.1 84.45) (end 138 84.45) (width 0.25) (layer "B.Cu") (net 2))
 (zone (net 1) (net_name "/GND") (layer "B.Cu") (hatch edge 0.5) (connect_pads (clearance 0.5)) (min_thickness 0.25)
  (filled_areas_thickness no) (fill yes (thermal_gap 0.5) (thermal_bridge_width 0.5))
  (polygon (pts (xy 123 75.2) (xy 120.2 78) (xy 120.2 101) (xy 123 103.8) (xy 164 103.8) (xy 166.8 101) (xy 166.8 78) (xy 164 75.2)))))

